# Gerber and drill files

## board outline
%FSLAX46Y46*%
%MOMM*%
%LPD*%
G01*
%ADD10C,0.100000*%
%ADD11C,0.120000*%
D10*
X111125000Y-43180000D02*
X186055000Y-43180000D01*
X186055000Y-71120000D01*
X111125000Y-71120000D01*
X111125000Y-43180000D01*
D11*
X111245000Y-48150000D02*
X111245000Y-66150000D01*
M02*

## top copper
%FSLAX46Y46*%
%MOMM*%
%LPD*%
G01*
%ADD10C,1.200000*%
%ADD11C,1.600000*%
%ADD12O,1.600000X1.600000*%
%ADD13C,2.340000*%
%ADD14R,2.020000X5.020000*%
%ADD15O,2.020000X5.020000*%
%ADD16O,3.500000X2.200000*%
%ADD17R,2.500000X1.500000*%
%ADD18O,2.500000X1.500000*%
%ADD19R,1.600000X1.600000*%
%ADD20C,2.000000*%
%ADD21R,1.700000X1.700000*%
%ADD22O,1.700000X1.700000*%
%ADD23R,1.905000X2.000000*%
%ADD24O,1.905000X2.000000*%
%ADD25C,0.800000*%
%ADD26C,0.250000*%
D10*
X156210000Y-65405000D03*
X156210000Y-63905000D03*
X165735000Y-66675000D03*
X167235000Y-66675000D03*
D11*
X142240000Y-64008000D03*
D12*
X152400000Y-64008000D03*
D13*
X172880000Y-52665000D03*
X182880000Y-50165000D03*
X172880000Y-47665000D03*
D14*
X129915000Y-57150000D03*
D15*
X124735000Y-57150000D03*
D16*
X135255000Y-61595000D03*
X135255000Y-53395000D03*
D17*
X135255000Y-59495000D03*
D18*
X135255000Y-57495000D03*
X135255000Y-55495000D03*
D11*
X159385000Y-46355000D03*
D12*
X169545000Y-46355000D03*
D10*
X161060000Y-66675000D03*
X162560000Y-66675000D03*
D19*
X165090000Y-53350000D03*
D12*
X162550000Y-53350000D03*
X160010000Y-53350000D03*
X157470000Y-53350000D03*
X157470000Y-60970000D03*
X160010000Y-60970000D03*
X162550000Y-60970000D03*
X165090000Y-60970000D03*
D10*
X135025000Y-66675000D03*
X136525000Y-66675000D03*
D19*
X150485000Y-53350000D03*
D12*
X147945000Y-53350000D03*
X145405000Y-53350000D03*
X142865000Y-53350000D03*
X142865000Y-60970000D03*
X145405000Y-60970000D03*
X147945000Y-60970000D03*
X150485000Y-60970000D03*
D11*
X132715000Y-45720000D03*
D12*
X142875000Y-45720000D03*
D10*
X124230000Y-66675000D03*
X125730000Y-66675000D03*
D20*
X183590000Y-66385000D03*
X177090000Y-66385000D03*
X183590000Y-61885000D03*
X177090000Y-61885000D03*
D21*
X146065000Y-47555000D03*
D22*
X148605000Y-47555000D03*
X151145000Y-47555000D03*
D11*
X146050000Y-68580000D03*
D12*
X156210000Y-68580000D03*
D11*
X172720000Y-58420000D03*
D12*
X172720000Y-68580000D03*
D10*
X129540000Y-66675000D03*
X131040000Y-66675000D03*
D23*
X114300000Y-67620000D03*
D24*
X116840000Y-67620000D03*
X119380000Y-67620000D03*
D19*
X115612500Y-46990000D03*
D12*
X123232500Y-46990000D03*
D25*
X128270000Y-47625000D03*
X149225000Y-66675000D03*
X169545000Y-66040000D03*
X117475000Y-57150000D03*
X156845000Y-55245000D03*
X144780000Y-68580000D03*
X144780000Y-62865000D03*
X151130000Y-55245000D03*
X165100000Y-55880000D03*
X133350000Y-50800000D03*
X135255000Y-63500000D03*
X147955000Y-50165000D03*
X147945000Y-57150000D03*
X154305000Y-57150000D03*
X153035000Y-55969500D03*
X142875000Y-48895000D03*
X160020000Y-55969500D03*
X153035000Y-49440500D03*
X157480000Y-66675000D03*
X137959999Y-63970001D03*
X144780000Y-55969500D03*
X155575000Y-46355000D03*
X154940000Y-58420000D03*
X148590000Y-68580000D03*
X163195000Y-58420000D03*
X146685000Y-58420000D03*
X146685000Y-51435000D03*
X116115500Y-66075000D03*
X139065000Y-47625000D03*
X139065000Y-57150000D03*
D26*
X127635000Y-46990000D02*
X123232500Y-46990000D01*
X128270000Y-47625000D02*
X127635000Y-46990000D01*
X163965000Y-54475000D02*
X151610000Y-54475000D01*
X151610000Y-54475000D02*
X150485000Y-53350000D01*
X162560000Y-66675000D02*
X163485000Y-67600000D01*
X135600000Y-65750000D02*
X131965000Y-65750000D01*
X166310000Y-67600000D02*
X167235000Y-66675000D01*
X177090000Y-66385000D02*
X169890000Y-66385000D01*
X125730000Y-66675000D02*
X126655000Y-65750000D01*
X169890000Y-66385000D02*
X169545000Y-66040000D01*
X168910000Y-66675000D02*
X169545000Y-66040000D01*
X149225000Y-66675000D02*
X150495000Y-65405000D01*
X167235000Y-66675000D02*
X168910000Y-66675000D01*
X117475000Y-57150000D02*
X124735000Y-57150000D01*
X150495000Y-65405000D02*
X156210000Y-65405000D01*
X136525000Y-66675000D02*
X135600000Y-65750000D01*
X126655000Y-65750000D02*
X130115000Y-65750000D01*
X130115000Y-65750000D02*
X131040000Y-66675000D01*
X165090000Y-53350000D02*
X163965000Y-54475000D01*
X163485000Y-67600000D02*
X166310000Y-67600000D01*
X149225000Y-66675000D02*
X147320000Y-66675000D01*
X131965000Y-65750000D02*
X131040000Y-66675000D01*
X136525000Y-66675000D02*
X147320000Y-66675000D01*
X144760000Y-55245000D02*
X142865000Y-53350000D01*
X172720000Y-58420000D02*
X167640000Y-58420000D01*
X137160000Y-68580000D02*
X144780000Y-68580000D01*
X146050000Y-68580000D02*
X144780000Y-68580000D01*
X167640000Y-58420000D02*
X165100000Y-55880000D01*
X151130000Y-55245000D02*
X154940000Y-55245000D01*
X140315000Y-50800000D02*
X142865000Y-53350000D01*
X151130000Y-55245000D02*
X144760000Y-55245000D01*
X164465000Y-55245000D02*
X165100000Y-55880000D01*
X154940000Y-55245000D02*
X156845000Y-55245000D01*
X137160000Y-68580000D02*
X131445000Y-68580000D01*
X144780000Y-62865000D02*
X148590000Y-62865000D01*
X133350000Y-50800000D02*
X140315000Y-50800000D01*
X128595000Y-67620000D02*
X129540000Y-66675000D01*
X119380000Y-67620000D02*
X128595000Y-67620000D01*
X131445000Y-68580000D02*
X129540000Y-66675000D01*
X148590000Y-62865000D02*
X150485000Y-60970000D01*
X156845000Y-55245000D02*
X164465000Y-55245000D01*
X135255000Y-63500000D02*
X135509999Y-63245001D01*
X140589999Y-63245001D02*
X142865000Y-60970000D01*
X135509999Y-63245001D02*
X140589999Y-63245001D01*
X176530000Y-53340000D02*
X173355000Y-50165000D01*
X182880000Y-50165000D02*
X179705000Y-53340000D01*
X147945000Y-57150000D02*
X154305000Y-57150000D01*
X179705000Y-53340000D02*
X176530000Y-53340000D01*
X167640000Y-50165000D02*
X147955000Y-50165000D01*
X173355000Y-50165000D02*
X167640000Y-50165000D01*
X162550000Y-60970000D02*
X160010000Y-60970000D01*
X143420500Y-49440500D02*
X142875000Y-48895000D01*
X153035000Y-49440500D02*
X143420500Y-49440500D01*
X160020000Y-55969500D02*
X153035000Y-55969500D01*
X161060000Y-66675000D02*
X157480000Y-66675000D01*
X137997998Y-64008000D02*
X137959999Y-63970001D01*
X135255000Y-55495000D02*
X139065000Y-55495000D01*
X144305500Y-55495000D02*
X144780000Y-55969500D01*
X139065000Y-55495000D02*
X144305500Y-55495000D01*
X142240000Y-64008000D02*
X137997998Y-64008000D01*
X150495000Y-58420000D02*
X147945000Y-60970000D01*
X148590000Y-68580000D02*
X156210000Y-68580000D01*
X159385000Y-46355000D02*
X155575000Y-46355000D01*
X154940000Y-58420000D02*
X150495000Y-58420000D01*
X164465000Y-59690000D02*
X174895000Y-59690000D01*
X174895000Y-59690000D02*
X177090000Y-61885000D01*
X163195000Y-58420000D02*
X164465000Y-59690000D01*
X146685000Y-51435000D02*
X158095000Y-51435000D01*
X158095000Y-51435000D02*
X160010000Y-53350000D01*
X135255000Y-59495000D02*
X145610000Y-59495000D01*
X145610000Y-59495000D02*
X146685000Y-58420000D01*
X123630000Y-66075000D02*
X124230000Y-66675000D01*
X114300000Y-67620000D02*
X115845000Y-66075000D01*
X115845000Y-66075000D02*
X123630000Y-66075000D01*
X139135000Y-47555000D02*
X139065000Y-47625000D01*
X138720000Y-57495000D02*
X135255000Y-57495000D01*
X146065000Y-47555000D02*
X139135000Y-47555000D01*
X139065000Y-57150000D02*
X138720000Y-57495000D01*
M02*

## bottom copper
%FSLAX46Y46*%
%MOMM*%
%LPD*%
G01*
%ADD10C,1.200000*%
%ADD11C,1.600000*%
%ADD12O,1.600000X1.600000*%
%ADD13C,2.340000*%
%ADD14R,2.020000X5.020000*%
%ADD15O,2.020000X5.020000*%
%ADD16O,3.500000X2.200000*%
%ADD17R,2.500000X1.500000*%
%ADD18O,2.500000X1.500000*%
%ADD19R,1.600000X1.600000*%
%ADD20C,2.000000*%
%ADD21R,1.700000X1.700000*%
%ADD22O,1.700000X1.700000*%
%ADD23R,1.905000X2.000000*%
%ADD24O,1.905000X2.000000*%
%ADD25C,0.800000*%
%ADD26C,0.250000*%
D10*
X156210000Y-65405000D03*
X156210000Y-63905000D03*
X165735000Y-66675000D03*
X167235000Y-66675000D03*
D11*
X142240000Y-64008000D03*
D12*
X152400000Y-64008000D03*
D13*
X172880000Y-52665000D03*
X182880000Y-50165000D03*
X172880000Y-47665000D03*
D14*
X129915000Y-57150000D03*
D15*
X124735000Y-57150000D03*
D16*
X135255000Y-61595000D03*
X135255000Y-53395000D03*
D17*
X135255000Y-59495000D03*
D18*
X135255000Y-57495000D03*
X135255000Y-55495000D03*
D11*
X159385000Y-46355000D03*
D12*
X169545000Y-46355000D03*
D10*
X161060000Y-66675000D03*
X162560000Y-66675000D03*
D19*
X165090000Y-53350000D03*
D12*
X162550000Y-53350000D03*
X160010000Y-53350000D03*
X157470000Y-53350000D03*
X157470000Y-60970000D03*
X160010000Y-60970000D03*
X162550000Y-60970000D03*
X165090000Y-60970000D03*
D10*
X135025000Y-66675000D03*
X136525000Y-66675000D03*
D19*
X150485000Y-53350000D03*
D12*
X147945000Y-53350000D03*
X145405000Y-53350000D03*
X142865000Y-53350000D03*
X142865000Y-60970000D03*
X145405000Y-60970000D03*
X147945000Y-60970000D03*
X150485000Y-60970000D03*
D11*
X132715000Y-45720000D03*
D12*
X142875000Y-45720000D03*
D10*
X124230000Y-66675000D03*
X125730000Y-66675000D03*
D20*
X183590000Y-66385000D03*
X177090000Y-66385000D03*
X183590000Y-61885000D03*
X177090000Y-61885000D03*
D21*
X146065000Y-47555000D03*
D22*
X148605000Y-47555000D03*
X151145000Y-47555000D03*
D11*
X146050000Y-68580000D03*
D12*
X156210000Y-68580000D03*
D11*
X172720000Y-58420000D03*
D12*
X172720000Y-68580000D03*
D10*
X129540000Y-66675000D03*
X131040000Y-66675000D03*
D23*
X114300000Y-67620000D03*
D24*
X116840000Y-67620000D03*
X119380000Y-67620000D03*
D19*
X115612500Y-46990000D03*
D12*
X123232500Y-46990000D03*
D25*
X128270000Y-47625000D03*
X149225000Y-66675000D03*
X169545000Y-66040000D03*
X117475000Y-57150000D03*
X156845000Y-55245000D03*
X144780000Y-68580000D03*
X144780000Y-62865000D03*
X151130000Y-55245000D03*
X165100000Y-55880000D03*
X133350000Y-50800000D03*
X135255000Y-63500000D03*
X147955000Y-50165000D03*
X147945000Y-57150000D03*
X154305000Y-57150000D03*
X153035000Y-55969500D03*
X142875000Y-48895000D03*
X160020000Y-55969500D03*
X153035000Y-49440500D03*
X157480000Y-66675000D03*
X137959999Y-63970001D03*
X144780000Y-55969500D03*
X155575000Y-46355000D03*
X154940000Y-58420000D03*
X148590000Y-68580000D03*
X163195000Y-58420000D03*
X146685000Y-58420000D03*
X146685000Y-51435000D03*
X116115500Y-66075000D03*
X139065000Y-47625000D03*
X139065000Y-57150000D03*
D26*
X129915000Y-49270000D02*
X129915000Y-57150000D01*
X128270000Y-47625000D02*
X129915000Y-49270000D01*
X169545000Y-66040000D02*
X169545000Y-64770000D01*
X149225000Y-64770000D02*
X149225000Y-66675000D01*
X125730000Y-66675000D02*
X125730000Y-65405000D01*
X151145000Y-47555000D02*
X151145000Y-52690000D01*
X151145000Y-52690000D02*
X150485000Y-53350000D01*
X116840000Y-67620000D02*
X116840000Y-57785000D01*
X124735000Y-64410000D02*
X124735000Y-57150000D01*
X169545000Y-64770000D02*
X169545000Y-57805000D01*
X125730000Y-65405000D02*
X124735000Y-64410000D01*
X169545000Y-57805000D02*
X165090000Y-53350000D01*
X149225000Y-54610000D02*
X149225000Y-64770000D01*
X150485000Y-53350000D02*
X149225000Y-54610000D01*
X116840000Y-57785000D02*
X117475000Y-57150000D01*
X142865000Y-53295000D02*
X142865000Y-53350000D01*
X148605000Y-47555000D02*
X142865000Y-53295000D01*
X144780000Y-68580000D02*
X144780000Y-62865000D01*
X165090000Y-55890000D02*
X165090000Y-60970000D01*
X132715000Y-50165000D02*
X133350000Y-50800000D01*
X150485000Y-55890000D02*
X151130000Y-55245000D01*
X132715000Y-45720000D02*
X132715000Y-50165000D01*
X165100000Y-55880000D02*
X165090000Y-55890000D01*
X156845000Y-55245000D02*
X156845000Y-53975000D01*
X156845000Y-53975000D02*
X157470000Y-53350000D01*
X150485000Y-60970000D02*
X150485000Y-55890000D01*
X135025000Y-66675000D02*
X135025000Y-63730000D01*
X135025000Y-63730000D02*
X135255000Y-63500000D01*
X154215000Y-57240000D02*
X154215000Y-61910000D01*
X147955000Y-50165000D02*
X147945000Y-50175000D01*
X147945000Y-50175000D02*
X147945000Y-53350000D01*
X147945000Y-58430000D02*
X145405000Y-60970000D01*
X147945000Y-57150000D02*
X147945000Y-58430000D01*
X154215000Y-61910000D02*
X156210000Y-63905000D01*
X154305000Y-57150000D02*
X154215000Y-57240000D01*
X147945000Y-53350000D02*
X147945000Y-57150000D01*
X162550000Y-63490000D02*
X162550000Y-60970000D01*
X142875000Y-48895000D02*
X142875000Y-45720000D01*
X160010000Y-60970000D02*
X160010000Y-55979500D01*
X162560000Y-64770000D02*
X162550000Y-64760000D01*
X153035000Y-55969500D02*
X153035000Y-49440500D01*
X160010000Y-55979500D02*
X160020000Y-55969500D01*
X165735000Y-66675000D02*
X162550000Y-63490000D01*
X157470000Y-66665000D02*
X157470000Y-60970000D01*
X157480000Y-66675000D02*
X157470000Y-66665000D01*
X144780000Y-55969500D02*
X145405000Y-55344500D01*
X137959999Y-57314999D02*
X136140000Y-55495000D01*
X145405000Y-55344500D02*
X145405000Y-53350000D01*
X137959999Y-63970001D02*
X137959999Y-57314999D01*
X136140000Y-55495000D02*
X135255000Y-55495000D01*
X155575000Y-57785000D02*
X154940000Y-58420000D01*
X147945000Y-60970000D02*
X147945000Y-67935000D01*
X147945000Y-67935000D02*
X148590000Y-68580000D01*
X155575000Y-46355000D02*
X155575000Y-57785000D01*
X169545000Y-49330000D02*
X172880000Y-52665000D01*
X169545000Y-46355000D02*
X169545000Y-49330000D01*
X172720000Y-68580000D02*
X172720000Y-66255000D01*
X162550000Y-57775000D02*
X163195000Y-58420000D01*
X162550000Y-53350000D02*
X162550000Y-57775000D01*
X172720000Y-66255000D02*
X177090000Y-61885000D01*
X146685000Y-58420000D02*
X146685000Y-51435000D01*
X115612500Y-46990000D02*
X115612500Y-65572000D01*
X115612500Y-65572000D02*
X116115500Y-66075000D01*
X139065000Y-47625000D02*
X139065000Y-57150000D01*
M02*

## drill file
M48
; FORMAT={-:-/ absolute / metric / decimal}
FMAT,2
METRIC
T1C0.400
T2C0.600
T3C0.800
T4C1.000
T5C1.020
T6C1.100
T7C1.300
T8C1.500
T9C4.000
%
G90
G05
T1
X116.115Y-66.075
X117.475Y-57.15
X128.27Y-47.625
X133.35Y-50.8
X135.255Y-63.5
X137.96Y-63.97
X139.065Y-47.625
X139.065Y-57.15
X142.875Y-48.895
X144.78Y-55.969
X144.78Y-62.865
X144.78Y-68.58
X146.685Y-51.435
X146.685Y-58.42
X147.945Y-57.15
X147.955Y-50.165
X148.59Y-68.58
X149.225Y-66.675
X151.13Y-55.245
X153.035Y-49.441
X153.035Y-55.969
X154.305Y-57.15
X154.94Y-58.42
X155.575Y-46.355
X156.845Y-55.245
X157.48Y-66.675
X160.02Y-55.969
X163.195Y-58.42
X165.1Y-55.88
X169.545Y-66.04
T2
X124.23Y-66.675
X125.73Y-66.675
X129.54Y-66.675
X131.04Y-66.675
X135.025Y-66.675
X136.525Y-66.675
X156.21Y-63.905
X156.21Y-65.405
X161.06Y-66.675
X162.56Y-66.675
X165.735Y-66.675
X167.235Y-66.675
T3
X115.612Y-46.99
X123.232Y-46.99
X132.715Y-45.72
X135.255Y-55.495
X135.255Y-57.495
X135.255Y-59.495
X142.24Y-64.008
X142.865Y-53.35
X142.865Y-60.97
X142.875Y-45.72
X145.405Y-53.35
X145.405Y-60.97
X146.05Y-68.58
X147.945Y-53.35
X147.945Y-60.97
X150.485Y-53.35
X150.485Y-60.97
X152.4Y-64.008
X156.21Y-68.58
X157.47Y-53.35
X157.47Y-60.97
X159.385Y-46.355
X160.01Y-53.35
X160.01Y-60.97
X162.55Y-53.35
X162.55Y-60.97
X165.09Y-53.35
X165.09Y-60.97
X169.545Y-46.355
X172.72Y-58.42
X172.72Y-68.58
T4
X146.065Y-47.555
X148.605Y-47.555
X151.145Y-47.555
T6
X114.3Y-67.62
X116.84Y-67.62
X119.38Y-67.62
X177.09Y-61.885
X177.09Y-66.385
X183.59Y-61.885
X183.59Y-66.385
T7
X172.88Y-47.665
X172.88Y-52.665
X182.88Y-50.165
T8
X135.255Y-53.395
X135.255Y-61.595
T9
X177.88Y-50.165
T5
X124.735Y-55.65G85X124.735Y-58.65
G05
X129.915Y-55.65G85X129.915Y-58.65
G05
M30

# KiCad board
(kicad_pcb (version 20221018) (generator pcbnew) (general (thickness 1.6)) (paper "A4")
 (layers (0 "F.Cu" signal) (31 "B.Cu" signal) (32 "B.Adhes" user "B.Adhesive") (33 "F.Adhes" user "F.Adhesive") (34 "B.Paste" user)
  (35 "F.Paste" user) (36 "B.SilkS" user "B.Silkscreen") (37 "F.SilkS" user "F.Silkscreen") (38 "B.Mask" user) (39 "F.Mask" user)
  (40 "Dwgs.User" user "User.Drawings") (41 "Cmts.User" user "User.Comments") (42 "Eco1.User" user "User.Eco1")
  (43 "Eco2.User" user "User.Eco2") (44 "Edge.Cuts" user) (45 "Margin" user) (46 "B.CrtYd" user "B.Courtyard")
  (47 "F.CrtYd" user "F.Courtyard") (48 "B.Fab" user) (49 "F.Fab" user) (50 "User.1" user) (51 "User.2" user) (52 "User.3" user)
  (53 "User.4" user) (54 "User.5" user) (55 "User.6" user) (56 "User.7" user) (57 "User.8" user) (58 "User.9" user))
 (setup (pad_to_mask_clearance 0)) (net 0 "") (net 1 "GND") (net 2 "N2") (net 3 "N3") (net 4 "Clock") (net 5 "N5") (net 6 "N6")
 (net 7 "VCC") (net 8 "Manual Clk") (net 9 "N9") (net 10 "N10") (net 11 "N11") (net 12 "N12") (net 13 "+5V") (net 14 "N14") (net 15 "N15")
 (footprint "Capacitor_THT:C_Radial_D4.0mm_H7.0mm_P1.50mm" (layer "F.Cu") (at 156.21 65.405 90)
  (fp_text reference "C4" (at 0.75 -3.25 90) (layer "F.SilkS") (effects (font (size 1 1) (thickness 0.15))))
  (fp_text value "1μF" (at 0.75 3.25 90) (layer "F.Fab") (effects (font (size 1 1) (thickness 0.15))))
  (pad "1" thru_hole circle (at 0 0 90) (size 1.2 1.2) (drill 0.6) (layers "*.Cu" "*.Mask") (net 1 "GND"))
  (pad "2" thru_hole circle (at 1.5 0 90) (size 1.2 1.2) (drill 0.6) (layers "*.Cu" "*.Mask") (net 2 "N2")))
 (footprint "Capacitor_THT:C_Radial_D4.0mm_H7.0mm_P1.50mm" (layer "F.Cu") (at 165.735 66.675)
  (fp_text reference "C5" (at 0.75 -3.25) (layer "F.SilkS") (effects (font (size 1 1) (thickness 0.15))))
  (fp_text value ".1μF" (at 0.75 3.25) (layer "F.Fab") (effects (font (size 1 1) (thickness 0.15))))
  (pad "1" thru_hole circle (at 0 0) (size 1.2 1.2) (drill 0.6) (layers "*.Cu" "*.Mask") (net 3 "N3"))
  (pad "2" thru_hole circle (at 1.5 0) (size 1.2 1.2) (drill 0.6) (layers "*.Cu" "*.Mask") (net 1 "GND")))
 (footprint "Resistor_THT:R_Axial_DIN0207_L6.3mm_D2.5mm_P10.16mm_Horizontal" (layer "F.Cu") (at 142.24 64.008)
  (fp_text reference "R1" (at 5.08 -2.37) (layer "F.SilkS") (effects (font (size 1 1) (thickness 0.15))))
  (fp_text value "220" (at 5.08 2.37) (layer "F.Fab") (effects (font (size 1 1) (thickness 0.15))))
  (pad "1" thru_hole circle (at 0 0) (size 1.6 1.6) (drill 0.8) (layers "*.Cu" "*.Mask") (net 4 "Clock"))
  (pad "2" thru_hole oval (at 10.16 0) (size 1.6 1.6) (drill 0.8) (layers "*.Cu" "*.Mask") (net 1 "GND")))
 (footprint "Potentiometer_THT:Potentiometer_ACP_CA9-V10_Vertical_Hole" (layer "F.Cu") (at 172.88 52.665)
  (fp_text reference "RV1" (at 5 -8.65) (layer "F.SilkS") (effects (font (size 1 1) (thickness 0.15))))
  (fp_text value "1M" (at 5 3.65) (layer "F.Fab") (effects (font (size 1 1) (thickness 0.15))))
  (pad "" np_thru_hole circle (at 5 -2.5) (size 4 4) (drill 4) (layers "*.Cu" "*.Mask"))
  (pad "1" thru_hole circle (at 0 0) (size 2.34 2.34) (drill 1.3) (layers "*.Cu" "*.Mask") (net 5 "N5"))
  (pad "2" thru_hole circle (at 10 -2.5) (size 2.34 2.34) (drill 1.3) (layers "*.Cu" "*.Mask") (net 2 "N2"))
  (pad "3" thru_hole circle (at 0 -5) (size 2.34 2.34) (drill 1.3) (layers "*.Cu" "*.Mask") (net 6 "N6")))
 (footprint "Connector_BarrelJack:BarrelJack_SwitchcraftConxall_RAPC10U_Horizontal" (layer "F.Cu") (at 129.915 57.15)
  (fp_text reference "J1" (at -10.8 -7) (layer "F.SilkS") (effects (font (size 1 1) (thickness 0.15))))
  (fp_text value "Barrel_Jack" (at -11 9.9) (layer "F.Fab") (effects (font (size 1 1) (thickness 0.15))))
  (fp_line (start -18.67 -9) (end -18.67 9) (stroke (width 0.12) (type solid)) (layer "Edge.Cuts"))
  (pad "1" thru_hole rect (at 0 0) (size 2.02 5.02) (drill oval 1.02 4.02) (layers "*.Cu" "*.Mask") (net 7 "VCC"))
  (pad "2" thru_hole oval (at -5.18 0) (size 2.02 5.02) (drill oval 1.02 4.02) (layers "*.Cu" "*.Mask") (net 1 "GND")))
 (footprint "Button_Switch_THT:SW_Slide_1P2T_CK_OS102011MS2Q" (layer "F.Cu") (at 135.255 59.495 90)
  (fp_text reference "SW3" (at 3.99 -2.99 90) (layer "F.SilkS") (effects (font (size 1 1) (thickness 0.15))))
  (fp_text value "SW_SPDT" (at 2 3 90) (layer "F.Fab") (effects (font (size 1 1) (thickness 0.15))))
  (pad "" thru_hole oval (at -2.1 0 90) (size 2.2 3.5) (drill 1.5) (layers "*.Cu" "*.Mask"))
  (pad "" thru_hole oval (at 6.1 0 90) (size 2.2 3.5) (drill 1.5) (layers "*.Cu" "*.Mask"))
  (pad "1" thru_hole rect (at 0 0 90) (size 1.5 2.5) (drill 0.8) (layers "*.Cu" "*.Mask") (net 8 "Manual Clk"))
  (pad "2" thru_hole oval (at 2 0 90) (size 1.5 2.5) (drill 0.8) (layers "*.Cu" "*.Mask") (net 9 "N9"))
  (pad "3" thru_hole oval (at 4 0 90) (size 1.5 2.5) (drill 0.8) (layers "*.Cu" "*.Mask") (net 4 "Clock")))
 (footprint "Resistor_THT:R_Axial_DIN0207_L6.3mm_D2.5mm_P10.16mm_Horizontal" (layer "F.Cu") (at 159.385 46.355)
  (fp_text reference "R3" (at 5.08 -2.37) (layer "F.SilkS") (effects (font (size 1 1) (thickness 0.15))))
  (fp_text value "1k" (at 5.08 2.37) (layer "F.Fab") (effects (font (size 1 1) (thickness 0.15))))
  (pad "1" thru_hole circle (at 0 0) (size 1.6 1.6) (drill 0.8) (layers "*.Cu" "*.Mask") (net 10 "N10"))
  (pad "2" thru_hole oval (at 10.16 0) (size 1.6 1.6) (drill 0.8) (layers "*.Cu" "*.Mask") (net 5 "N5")))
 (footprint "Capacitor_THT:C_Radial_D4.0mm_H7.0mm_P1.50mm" (layer "F.Cu") (at 161.06 66.675)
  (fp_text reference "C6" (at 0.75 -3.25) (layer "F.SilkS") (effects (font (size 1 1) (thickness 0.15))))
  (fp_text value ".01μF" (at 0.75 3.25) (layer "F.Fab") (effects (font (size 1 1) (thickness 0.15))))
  (pad "1" thru_hole circle (at 0 0) (size 1.2 1.2) (drill 0.6) (layers "*.Cu" "*.Mask") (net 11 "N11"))
  (pad "2" thru_hole circle (at 1.5 0) (size 1.2 1.2) (drill 0.6) (layers "*.Cu" "*.Mask") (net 1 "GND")))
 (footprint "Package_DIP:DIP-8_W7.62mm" (layer "F.Cu") (at 165.09 53.35 -90)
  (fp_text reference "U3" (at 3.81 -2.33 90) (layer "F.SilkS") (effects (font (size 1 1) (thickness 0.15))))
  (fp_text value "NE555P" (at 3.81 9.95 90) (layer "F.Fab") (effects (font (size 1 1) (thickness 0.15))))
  (pad "1" thru_hole rect (at 0 0 270) (size 1.6 1.6) (drill 0.8) (layers "*.Cu" "*.Mask") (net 1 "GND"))
  (pad "2" thru_hole oval (at 0 2.54 270) (size 1.6 1.6) (drill 0.8) (layers "*.Cu" "*.Mask") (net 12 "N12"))
  (pad "3" thru_hole oval (at 0 5.08 270) (size 1.6 1.6) (drill 0.8) (layers "*.Cu" "*.Mask") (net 8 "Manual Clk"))
  (pad "4" thru_hole oval (at 0 7.62 270) (size 1.6 1.6) (drill 0.8) (layers "*.Cu" "*.Mask") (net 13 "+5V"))
  (pad "5" thru_hole oval (at 7.62 7.62 270) (size 1.6 1.6) (drill 0.8) (layers "*.Cu" "*.Mask") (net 11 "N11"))
  (pad "6" thru_hole oval (at 7.62 5.08 270) (size 1.6 1.6) (drill 0.8) (layers "*.Cu" "*.Mask") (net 3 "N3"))
  (pad "7" thru_hole oval (at 7.62 2.54 270) (size 1.6 1.6) (drill 0.8) (layers "*.Cu" "*.Mask") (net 3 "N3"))
  (pad "8" thru_hole oval (at 7.62 0 270) (size 1.6 1.6) (drill 0.8) (layers "*.Cu" "*.Mask") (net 13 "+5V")))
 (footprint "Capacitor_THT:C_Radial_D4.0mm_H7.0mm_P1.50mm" (layer "F.Cu") (at 135.025 66.675)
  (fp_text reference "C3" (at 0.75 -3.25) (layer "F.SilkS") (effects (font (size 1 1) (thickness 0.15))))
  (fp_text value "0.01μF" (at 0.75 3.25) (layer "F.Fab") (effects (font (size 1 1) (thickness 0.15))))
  (pad "1" thru_hole circle (at 0 0) (size 1.2 1.2) (drill 0.6) (layers "*.Cu" "*.Mask") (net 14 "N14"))
  (pad "2" thru_hole circle (at 1.5 0) (size 1.2 1.2) (drill 0.6) (layers "*.Cu" "*.Mask") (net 1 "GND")))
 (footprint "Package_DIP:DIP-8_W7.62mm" (layer "F.Cu") (at 150.485 53.35 -90)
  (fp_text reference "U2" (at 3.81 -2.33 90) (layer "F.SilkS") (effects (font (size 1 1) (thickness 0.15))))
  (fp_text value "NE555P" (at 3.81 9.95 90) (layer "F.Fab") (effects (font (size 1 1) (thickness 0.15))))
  (pad "1" thru_hole rect (at 0 0 270) (size 1.6 1.6) (drill 0.8) (layers "*.Cu" "*.Mask") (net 1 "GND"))
  (pad "2" thru_hole oval (at 0 2.54 270) (size 1.6 1.6) (drill 0.8) (layers "*.Cu" "*.Mask") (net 2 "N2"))
  (pad "3" thru_hole oval (at 0 5.08 270) (size 1.6 1.6) (drill 0.8) (layers "*.Cu" "*.Mask") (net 4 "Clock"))
  (pad "4" thru_hole oval (at 0 7.62 270) (size 1.6 1.6) (drill 0.8) (layers "*.Cu" "*.Mask") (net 13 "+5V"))
  (pad "5" thru_hole oval (at 7.62 7.62 270) (size 1.6 1.6) (drill 0.8) (layers "*.Cu" "*.Mask") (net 14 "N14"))
  (pad "6" thru_hole oval (at 7.62 5.08 270) (size 1.6 1.6) (drill 0.8) (layers "*.Cu" "*.Mask") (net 2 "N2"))
  (pad "7" thru_hole oval (at 7.62 2.54 270) (size 1.6 1.6) (drill 0.8) (layers "*.Cu" "*.Mask") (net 10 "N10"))
  (pad "8" thru_hole oval (at 7.62 0 270) (size 1.6 1.6) (drill 0.8) (layers "*.Cu" "*.Mask") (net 13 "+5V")))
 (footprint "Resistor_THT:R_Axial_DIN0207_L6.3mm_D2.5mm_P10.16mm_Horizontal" (layer "F.Cu") (at 132.715 45.72)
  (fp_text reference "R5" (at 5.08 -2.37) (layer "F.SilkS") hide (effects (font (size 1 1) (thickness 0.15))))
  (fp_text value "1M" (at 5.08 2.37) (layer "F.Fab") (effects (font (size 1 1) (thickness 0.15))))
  (pad "1" thru_hole circle (at 0 0) (size 1.6 1.6) (drill 0.8) (layers "*.Cu" "*.Mask") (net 13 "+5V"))
  (pad "2" thru_hole oval (at 10.16 0) (size 1.6 1.6) (drill 0.8) (layers "*.Cu" "*.Mask") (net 3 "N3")))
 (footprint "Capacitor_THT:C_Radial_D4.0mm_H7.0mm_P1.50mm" (layer "F.Cu") (at 124.23 66.675)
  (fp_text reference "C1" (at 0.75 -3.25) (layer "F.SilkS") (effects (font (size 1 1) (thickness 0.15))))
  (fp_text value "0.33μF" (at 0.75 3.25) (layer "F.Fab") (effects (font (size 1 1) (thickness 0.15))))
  (pad "1" thru_hole circle (at 0 0) (size 1.2 1.2) (drill 0.6) (layers "*.Cu" "*.Mask") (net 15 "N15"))
  (pad "2" thru_hole circle (at 1.5 0) (size 1.2 1.2) (drill 0.6) (layers "*.Cu" "*.Mask") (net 1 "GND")))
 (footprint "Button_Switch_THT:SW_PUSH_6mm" (layer "F.Cu") (at 183.59 66.385 180)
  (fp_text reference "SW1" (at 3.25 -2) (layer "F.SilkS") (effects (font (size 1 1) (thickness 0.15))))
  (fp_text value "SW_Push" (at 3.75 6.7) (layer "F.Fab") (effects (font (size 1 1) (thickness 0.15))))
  (pad "1" thru_hole circle (at 0 0 270) (size 2 2) (drill 1.1) (layers "*.Cu" "*.Mask") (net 1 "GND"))
  (pad "1" thru_hole circle (at 6.5 0 270) (size 2 2) (drill 1.1) (layers "*.Cu" "*.Mask") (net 1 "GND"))
  (pad "2" thru_hole circle (at 0 4.5 270) (size 2 2) (drill 1.1) (layers "*.Cu" "*.Mask") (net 12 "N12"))
  (pad "2" thru_hole circle (at 6.5 4.5 270) (size 2 2) (drill 1.1) (layers "*.Cu" "*.Mask") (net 12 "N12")))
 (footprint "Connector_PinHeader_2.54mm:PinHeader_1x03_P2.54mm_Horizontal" (layer "F.Cu") (at 146.065 47.555 90)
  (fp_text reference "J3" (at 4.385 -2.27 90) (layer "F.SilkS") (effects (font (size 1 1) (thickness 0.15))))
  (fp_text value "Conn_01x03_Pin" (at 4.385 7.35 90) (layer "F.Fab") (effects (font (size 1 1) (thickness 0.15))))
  (pad "1" thru_hole rect (at 0 0 90) (size 1.7 1.7) (drill 1) (layers "*.Cu" "*.Mask") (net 9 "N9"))
  (pad "2" thru_hole oval (at 0 2.54 90) (size 1.7 1.7) (drill 1) (layers "*.Cu" "*.Mask") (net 13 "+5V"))
  (pad "3" thru_hole oval (at 0 5.08 90) (size 1.7 1.7) (drill 1) (layers "*.Cu" "*.Mask") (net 1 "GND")))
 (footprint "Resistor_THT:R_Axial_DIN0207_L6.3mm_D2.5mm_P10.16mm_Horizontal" (layer "F.Cu") (at 146.05 68.58)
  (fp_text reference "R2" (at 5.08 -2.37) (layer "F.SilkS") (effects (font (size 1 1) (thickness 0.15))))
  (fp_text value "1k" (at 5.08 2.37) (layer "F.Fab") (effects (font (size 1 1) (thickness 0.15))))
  (pad "1" thru_hole circle (at 0 0) (size 1.6 1.6) (drill 0.8) (layers "*.Cu" "*.Mask") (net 13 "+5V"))
  (pad "2" thru_hole oval (at 10.16 0) (size 1.6 1.6) (drill 0.8) (layers "*.Cu" "*.Mask") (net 10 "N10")))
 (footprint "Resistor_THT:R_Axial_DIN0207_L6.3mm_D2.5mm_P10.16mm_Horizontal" (layer "F.Cu") (at 172.72 58.42 -90)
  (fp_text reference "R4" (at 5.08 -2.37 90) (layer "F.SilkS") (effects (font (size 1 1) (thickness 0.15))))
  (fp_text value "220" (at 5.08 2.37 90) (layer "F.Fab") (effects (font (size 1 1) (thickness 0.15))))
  (pad "1" thru_hole circle (at 0 0 270) (size 1.6 1.6) (drill 0.8) (layers "*.Cu" "*.Mask") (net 13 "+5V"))
  (pad "2" thru_hole oval (at 10.16 0 270) (size 1.6 1.6) (drill 0.8) (layers "*.Cu" "*.Mask") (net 12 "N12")))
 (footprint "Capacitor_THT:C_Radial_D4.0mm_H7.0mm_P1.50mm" (layer "F.Cu") (at 129.54 66.675)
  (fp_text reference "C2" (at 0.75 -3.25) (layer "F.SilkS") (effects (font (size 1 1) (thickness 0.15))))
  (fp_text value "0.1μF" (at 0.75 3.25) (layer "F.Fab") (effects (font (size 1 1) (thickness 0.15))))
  (pad "1" thru_hole circle (at 0 0) (size 1.2 1.2) (drill 0.6) (layers "*.Cu" "*.Mask") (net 13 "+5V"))
  (pad "2" thru_hole circle (at 1.5 0) (size 1.2 1.2) (drill 0.6) (layers "*.Cu" "*.Mask") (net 1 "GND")))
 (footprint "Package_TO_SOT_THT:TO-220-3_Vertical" (layer "F.Cu") (at 114.3 67.62)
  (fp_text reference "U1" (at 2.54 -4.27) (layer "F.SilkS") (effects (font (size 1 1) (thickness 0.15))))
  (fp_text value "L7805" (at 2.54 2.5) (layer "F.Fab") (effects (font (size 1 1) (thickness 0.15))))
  (pad "1" thru_hole rect (at 0 0) (size 1.905 2) (drill 1.1) (layers "*.Cu" "*.Mask") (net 15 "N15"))
  (pad "2" thru_hole oval (at 2.54 0) (size 1.905 2) (drill 1.1) (layers "*.Cu" "*.Mask") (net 1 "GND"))
  (pad "3" thru_hole oval (at 5.08 0) (size 1.905 2) (drill 1.1) (layers "*.Cu" "*.Mask") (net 13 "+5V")))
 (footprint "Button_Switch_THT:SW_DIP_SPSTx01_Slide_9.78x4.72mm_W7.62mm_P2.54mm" (layer "F.Cu") (at 115.6125 46.99)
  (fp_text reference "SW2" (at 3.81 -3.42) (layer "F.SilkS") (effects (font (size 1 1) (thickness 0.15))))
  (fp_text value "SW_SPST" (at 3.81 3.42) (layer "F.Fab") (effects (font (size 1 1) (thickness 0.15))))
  (pad "1" thru_hole rect (at 0 0) (size 1.6 1.6) (drill 0.8) (layers "*.Cu" "*.Mask") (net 15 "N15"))
  (pad "2" thru_hole oval (at 7.62 0) (size 1.6 1.6) (drill 0.8) (layers "*.Cu" "*.Mask") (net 7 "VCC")))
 (gr_rect (start 111.125 43.18) (end 186.055 71.12) (stroke (width 0.1) (type default)) (fill none) (layer "Edge.Cuts"))
 (segment (start 127.635 46.99) (end 123.2325 46.99) (width 0.25) (layer "F.Cu") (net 7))
 (segment (start 128.27 47.625) (end 127.635 46.99) (width 0.25) (layer "F.Cu") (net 7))
 (via (at 128.27 47.625) (size 0.8) (drill 0.4) (layers "F.Cu" "B.Cu") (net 7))
 (segment (start 129.915 49.27) (end 129.915 57.15) (width 0.25) (layer "B.Cu") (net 7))
 (segment (start 128.27 47.625) (end 129.915 49.27) (width 0.25) (layer "B.Cu") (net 7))
 (segment (start 163.965 54.475) (end 151.61 54.475) (width 0.25) (layer "F.Cu") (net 1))
 (segment (start 151.61 54.475) (end 150.485 53.35) (width 0.25) (layer "F.Cu") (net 1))
 (segment (start 162.56 66.675) (end 163.485 67.6) (width 0.25) (layer "F.Cu") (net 1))
 (segment (start 135.6 65.75) (end 131.965 65.75) (width 0.25) (layer "F.Cu") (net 1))
 (segment (start 166.31 67.6) (end 167.235 66.675) (width 0.25) (layer "F.Cu") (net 1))
 (segment (start 177.09 66.385) (end 169.89 66.385) (width 0.25) (layer "F.Cu") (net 1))
 (segment (start 125.73 66.675) (end 126.655 65.75) (width 0.25) (layer "F.Cu") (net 1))
 (segment (start 169.89 66.385) (end 169.545 66.04) (width 0.25) (layer "F.Cu") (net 1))
 (segment (start 168.91 66.675) (end 169.545 66.04) (width 0.25) (layer "F.Cu") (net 1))
 (segment (start 149.225 66.675) (end 150.495 65.405) (width 0.25) (layer "F.Cu") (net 1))
 (segment (start 167.235 66.675) (end 168.91 66.675) (width 0.25) (layer "F.Cu") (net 1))
 (segment (start 117.475 57.15) (end 124.735 57.15) (width 0.25) (layer "F.Cu") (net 1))
 (segment (start 150.495 65.405) (end 156.21 65.405) (width 0.25) (layer "F.Cu") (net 1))
 (segment (start 136.525 66.675) (end 135.6 65.75) (width 0.25) (layer "F.Cu") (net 1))
 (segment (start 126.655 65.75) (end 130.115 65.75) (width 0.25) (layer "F.Cu") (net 1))
 (segment (start 130.115 65.75) (end 131.04 66.675) (width 0.25) (layer "F.Cu") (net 1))
 (segment (start 165.09 53.35) (end 163.965 54.475) (width 0.25) (layer "F.Cu") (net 1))
 (segment (start 163.485 67.6) (end 166.31 67.6) (width 0.25) (layer "F.Cu") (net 1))
 (segment (start 149.225 66.675) (end 147.32 66.675) (width 0.25) (layer "F.Cu") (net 1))
 (segment (start 131.965 65.75) (end 131.04 66.675) (width 0.25) (layer "F.Cu") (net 1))
 (segment (start 136.525 66.675) (end 147.32 66.675) (width 0.25) (layer "F.Cu") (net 1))
 (via (at 149.225 66.675) (size 0.8) (drill 0.4) (layers "F.Cu" "B.Cu") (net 1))
 (via (at 169.545 66.04) (size 0.8) (drill 0.4) (layers "F.Cu" "B.Cu") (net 1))
 (via (at 117.475 57.15) (size 0.8) (drill 0.4) (layers "F.Cu" "B.Cu") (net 1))
 (segment (start 169.545 66.04) (end 169.545 64.77) (width 0.25) (layer "B.Cu") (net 1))
 (segment (start 149.225 64.77) (end 149.225 66.675) (width 0.25) (layer "B.Cu") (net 1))
 (segment (start 125.73 66.675) (end 125.73 65.405) (width 0.25) (layer "B.Cu") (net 1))
 (segment (start 151.145 47.555) (end 151.145 52.69) (width 0.25) (layer "B.Cu") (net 1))
 (segment (start 151.145 52.69) (end 150.485 53.35) (width 0.25) (layer "B.Cu") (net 1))
 (segment (start 116.84 67.62) (end 116.84 57.785) (width 0.25) (layer "B.Cu") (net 1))
 (segment (start 124.735 64.41) (end 124.735 57.15) (width 0.25) (layer "B.Cu") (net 1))
 (segment (start 169.545 64.77) (end 169.545 57.805) (width 0.25) (layer "B.Cu") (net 1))
 (segment (start 125.73 65.405) (end 124.735 64.41) (width 0.25) (layer "B.Cu") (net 1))
 (segment (start 169.545 57.805) (end 165.09 53.35) (width 0.25) (layer "B.Cu") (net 1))
 (segment (start 149.225 54.61) (end 149.225 64.77) (width 0.25) (layer "B.Cu") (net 1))
 (segment (start 150.485 53.35) (end 149.225 54.61) (width 0.25) (layer "B.Cu") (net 1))
 (segment (start 116.84 57.785) (end 117.475 57.15) (width 0.25) (layer "B.Cu") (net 1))
 (segment (start 144.76 55.245) (end 142.865 53.35) (width 0.25) (layer "F.Cu") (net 13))
 (segment (start 172.72 58.42) (end 167.64 58.42) (width 0.25) (layer "F.Cu") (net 13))
 (segment (start 137.16 68.58) (end 144.78 68.58) (width 0.25) (layer "F.Cu") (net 13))
 (segment (start 146.05 68.58) (end 144.78 68.58) (width 0.25) (layer "F.Cu") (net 13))
 (segment (start 167.64 58.42) (end 165.1 55.88) (width 0.25) (layer "F.Cu") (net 13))
 (segment (start 151.13 55.245) (end 154.94 55.245) (width 0.25) (layer "F.Cu") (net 13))
 (segment (start 140.315 50.8) (end 142.865 53.35) (width 0.25) (layer "F.Cu") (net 13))
 (segment (start 151.13 55.245) (end 144.76 55.245) (width 0.25) (layer "F.Cu") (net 13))
 (segment (start 164.465 55.245) (end 165.1 55.88) (width 0.25) (layer "F.Cu") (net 13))
 (segment (start 154.94 55.245) (end 156.845 55.245) (width 0.25) (layer "F.Cu") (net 13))
 (segment (start 137.16 68.58) (end 131.445 68.58) (width 0.25) (layer "F.Cu") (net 13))
 (segment (start 144.78 62.865) (end 148.59 62.865) (width 0.25) (layer "F.Cu") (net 13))
 (segment (start 133.35 50.8) (end 140.315 50.8) (width 0.25) (layer "F.Cu") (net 13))
 (segment (start 128.595 67.62) (end 129.54 66.675) (width 0.25) (layer "F.Cu") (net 13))
 (segment (start 119.38 67.62) (end 128.595 67.62) (width 0.25) (layer "F.Cu") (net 13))
 (segment (start 131.445 68.58) (end 129.54 66.675) (width 0.25) (layer "F.Cu") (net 13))
 (segment (start 148.59 62.865) (end 150.485 60.97) (width 0.25) (layer "F.Cu") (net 13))
 (segment (start 156.845 55.245) (end 164.465 55.245) (width 0.25) (layer "F.Cu") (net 13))
 (via (at 156.845 55.245) (size 0.8) (drill 0.4) (layers "F.Cu" "B.Cu") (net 13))
 (via (at 144.78 68.58) (size 0.8) (drill 0.4) (layers "F.Cu" "B.Cu") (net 13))
 (via (at 144.78 62.865) (size 0.8) (drill 0.4) (layers "F.Cu" "B.Cu") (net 13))
 (via (at 151.13 55.245) (size 0.8) (drill 0.4) (layers "F.Cu" "B.Cu") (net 13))
 (via (at 165.1 55.88) (size 0.8) (drill 0.4) (layers "F.Cu" "B.Cu") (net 13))
 (via (at 133.35 50.8) (size 0.8) (drill 0.4) (layers "F.Cu" "B.Cu") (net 13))
 (segment (start 142.865 53.295) (end 142.865 53.35) (width 0.25) (layer "B.Cu") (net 13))
 (segment (start 148.605 47.555) (end 142.865 53.295) (width 0.25) (layer "B.Cu") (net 13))
 (segment (start 144.78 68.58) (end 144.78 62.865) (width 0.25) (layer "B.Cu") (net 13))
 (segment (start 165.09 55.89) (end 165.09 60.97) (width 0.25) (layer "B.Cu") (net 13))
 (segment (start 132.715 50.165) (end 133.35 50.8) (width 0.25) (layer "B.Cu") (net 13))
 (segment (start 150.485 55.89) (end 151.13 55.245) (width 0.25) (layer "B.Cu") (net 13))
 (segment (start 132.715 45.72) (end 132.715 50.165) (width 0.25) (layer "B.Cu") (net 13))
 (segment (start 165.1 55.88) (end 165.09 55.89) (width 0.25) (layer "B.Cu") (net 13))
 (segment (start 156.845 55.245) (end 156.845 53.975) (width 0.25) (layer "B.Cu") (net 13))
 (segment (start 156.845 53.975) (end 157.47 53.35) (width 0.25) (layer "B.Cu") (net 13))
 (segment (start 150.485 60.97) (end 150.485 55.89) (width 0.25) (layer "B.Cu") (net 13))
 (segment (start 135.255 63.5) (end 135.509999 63.245001) (width 0.25) (layer "F.Cu") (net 14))
 (segment (start 140.589999 63.245001) (end 142.865 60.97) (width 0.25) (layer "F.Cu") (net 14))
 (segment (start 135.509999 63.245001) (end 140.589999 63.245001) (width 0.25) (layer "F.Cu") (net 14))
 (via (at 135.255 63.5) (size 0.8) (drill 0.4) (layers "F.Cu" "B.Cu") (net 14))
 (segment (start 135.025 66.675) (end 135.025 63.73) (width 0.25) (layer "B.Cu") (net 14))
 (segment (start 135.025 63.73) (end 135.255 63.5) (width 0.25) (layer "B.Cu") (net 14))
 (segment (start 176.53 53.34) (end 173.355 50.165) (width 0.25) (layer "F.Cu") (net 2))
 (segment (start 182.88 50.165) (end 179.705 53.34) (width 0.25) (layer "F.Cu") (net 2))
 (segment (start 147.945 57.15) (end 154.305 57.15) (width 0.25) (layer "F.Cu") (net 2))
 (segment (start 179.705 53.34) (end 176.53 53.34) (width 0.25) (layer "F.Cu") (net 2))
 (segment (start 167.64 50.165) (end 147.955 50.165) (width 0.25) (layer "F.Cu") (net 2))
 (segment (start 173.355 50.165) (end 167.64 50.165) (width 0.25) (layer "F.Cu") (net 2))
 (via (at 147.955 50.165) (size 0.8) (drill 0.4) (layers "F.Cu" "B.Cu") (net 2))
 (via (at 147.945 57.15) (size 0.8) (drill 0.4) (layers "F.Cu" "B.Cu") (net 2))
 (via (at 154.305 57.15) (size 0.8) (drill 0.4) (layers "F.Cu" "B.Cu") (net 2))
 (segment (start 154.215 57.24) (end 154.215 61.91) (width 0.25) (layer "B.Cu") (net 2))
 (segment (start 147.955 50.165) (end 147.945 50.175) (width 0.25) (layer "B.Cu") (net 2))
 (segment (start 147.945 50.175) (end 147.945 53.35) (width 0.25) (layer "B.Cu") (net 2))
 (segment (start 147.945 58.43) (end 145.405 60.97) (width 0.25) (layer "B.Cu") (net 2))
 (segment (start 147.945 57.15) (end 147.945 58.43) (width 0.25) (layer "B.Cu") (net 2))
 (segment (start 154.215 61.91) (end 156.21 63.905) (width 0.25) (layer "B.Cu") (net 2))
 (segment (start 154.305 57.15) (end 154.215 57.24) (width 0.25) (layer "B.Cu") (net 2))
 (segment (start 147.945 53.35) (end 147.945 57.15) (width 0.25) (layer "B.Cu") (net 2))
 (segment (start 162.55 60.97) (end 160.01 60.97) (width 0.25) (layer "F.Cu") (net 3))
 (segment (start 143.4205 49.4405) (end 142.875 48.895) (width 0.25) (layer "F.Cu") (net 3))
 (segment (start 153.035 49.4405) (end 143.4205 49.4405) (width 0.25) (layer "F.Cu") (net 3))
 (segment (start 160.02 55.9695) (end 153.035 55.9695) (width 0.25) (layer "F.Cu") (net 3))
 (via (at 153.035 55.9695) (size 0.8) (drill 0.4) (layers "F.Cu" "B.Cu") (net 3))
 (via (at 142.875 48.895) (size 0.8) (drill 0.4) (layers "F.Cu" "B.Cu") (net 3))
 (via (at 160.02 55.9695) (size 0.8) (drill 0.4) (layers "F.Cu" "B.Cu") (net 3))
 (via (at 153.035 49.4405) (size 0.8) (drill 0.4) (layers "F.Cu" "B.Cu") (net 3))
 (segment (start 162.55 63.49) (end 162.55 60.97) (width 0.25) (layer "B.Cu") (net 3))
 (segment (start 142.875 48.895) (end 142.875 45.72) (width 0.25) (layer "B.Cu") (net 3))
 (segment (start 160.01 60.97) (end 160.01 55.9795) (width 0.25) (layer "B.Cu") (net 3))
 (segment (start 162.56 64.77) (end 162.55 64.76) (width 0.25) (layer "B.Cu") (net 3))
 (segment (start 153.035 55.9695) (end 153.035 49.4405) (width 0.25) (layer "B.Cu") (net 3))
 (segment (start 160.01 55.9795) (end 160.02 55.9695) (width 0.25) (layer "B.Cu") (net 3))
 (segment (start 165.735 66.675) (end 162.55 63.49) (width 0.25) (layer "B.Cu") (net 3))
 (segment (start 161.06 66.675) (end 157.48 66.675) (width 0.25) (layer "F.Cu") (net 11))
 (via (at 157.48 66.675) (size 0.8) (drill 0.4) (layers "F.Cu" "B.Cu") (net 11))
 (segment (start 157.47 66.665) (end 157.47 60.97) (width 0.25) (layer "B.Cu") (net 11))
 (segment (start 157.48 66.675) (end 157.47 66.665) (width 0.25) (layer "B.Cu") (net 11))
 (segment (start 137.997998 64.008) (end 137.959999 63.970001) (width 0.25) (layer "F.Cu") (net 4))
 (segment (start 135.255 55.495) (end 139.065 55.495) (width 0.25) (layer "F.Cu") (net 4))
 (segment (start 144.3055 55.495) (end 144.78 55.9695) (width 0.25) (layer "F.Cu") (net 4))
 (segment (start 139.065 55.495) (end 144.3055 55.495) (width 0.25) (layer "F.Cu") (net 4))
 (segment (start 142.24 64.008) (end 137.997998 64.008) (width 0.25) (layer "F.Cu") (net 4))
 (via (at 137.959999 63.970001) (size 0.8) (drill 0.4) (layers "F.Cu" "B.Cu") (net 4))
 (via (at 144.78 55.9695) (size 0.8) (drill 0.4) (layers "F.Cu" "B.Cu") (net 4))
 (segment (start 144.78 55.9695) (end 145.405 55.3445) (width 0.25) (layer "B.Cu") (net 4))
 (segment (start 137.959999 57.314999) (end 136.14 55.495) (width 0.25) (layer "B.Cu") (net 4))
 (segment (start 145.405 55.3445) (end 145.405 53.35) (width 0.25) (layer "B.Cu") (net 4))
 (segment (start 137.959999 63.970001) (end 137.959999 57.314999) (width 0.25) (layer "B.Cu") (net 4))
 (segment (start 136.14 55.495) (end 135.255 55.495) (width 0.25) (layer "B.Cu") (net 4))
 (segment (start 150.495 58.42) (end 147.945 60.97) (width 0.25) (layer "F.Cu") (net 10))
 (segment (start 148.59 68.58) (end 156.21 68.58) (width 0.25) (layer "F.Cu") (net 10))
 (segment (start 159.385 46.355) (end 155.575 46.355) (width 0.25) (layer "F.Cu") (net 10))
 (segment (start 154.94 58.42) (end 150.495 58.42) (width 0.25) (layer "F.Cu") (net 10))
 (via (at 155.575 46.355) (size 0.8) (drill 0.4) (layers "F.Cu" "B.Cu") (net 10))
 (via (at 154.94 58.42) (size 0.8) (drill 0.4) (layers "F.Cu" "B.Cu") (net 10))
 (via (at 148.59 68.58) (size 0.8) (drill 0.4) (layers "F.Cu" "B.Cu") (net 10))
 (segment (start 155.575 57.785) (end 154.94 58.42) (width 0.25) (layer "B.Cu") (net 10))
 (segment (start 147.945 60.97) (end 147.945 67.935) (width 0.25) (layer "B.Cu") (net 10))
 (segment (start 147.945 67.935) (end 148.59 68.58) (width 0.25) (layer "B.Cu") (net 10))
 (segment (start 155.575 46.355) (end 155.575 57.785) (width 0.25) (layer "B.Cu") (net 10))
 (segment (start 169.545 49.33) (end 172.88 52.665) (width 0.25) (layer "B.Cu") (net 5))
 (segment (start 169.545 46.355) (end 169.545 49.33) (width 0.25) (layer "B.Cu") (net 5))
 (segment (start 164.465 59.69) (end 174.895 59.69) (width 0.25) (layer "F.Cu") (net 12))
 (segment (start 174.895 59.69) (end 177.09 61.885) (width 0.25) (layer "F.Cu") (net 12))
 (segment (start 163.195 58.42) (end 164.465 59.69) (width 0.25) (layer "F.Cu") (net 12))
 (via (at 163.195 58.42) (size 0.8) (drill 0.4) (layers "F.Cu" "B.Cu") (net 12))
 (segment (start 172.72 68.58) (end 172.72 66.255) (width 0.25) (layer "B.Cu") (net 12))
 (segment (start 162.55 57.775) (end 163.195 58.42) (width 0.25) (layer "B.Cu") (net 12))
 (segment (start 162.55 53.35) (end 162.55 57.775) (width 0.25) (layer "B.Cu") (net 12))
 (segment (start 172.72 66.255) (end 177.09 61.885) (width 0.25) (layer "B.Cu") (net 12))
 (segment (start 146.685 51.435) (end 158.095 51.435) (width 0.25) (layer "F.Cu") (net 8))
 (segment (start 158.095 51.435) (end 160.01 53.35) (width 0.25) (layer "F.Cu") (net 8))
 (segment (start 135.255 59.495) (end 145.61 59.495) (width 0.25) (layer "F.Cu") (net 8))
 (segment (start 145.61 59.495) (end 146.685 58.42) (width 0.25) (layer "F.Cu") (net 8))
 (via (at 146.685 58.42) (size 0.8) (drill 0.4) (layers "F.Cu" "B.Cu") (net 8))
 (via (at 146.685 51.435) (size 0.8) (drill 0.4) (layers "F.Cu" "B.Cu") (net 8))
 (segment (start 146.685 58.42) (end 146.685 51.435) (width 0.25) (layer "B.Cu") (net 8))
 (segment (start 123.63 66.075) (end 124.23 66.675) (width 0.25) (layer "F.Cu") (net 15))
 (segment (start 114.3 67.62) (end 115.845 66.075) (width 0.25) (layer "F.Cu") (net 15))
 (segment (start 115.845 66.075) (end 123.63 66.075) (width 0.25) (layer "F.Cu") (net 15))
 (via (at 116.1155 66.075) (size 0.8) (drill 0.4) (layers "F.Cu" "B.Cu") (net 15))
 (segment (start 115.6125 46.99) (end 115.6125 65.572) (width 0.25) (layer "B.Cu") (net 15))
 (segment (start 115.6125 65.572) (end 116.1155 66.075) (width 0.25) (layer "B.Cu") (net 15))
 (segment (start 139.135 47.555) (end 139.065 47.625) (width 0.25) (layer "F.Cu") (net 9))
 (segment (start 138.72 57.495) (end 135.255 57.495) (width 0.25) (layer "F.Cu") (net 9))
 (segment (start 146.065 47.555) (end 139.135 47.555) (width 0.25) (layer "F.Cu") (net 9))
 (segment (start 139.065 57.15) (end 138.72 57.495) (width 0.25) (layer "F.Cu") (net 9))
 (via (at 139.065 47.625) (size 0.8) (drill 0.4) (layers "F.Cu" "B.Cu") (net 9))
 (via (at 139.065 57.15) (size 0.8) (drill 0.4) (layers "F.Cu" "B.Cu") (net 9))
 (segment (start 139.065 47.625) (end 139.065 57.15) (width 0.25) (layer "B.Cu") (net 9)))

